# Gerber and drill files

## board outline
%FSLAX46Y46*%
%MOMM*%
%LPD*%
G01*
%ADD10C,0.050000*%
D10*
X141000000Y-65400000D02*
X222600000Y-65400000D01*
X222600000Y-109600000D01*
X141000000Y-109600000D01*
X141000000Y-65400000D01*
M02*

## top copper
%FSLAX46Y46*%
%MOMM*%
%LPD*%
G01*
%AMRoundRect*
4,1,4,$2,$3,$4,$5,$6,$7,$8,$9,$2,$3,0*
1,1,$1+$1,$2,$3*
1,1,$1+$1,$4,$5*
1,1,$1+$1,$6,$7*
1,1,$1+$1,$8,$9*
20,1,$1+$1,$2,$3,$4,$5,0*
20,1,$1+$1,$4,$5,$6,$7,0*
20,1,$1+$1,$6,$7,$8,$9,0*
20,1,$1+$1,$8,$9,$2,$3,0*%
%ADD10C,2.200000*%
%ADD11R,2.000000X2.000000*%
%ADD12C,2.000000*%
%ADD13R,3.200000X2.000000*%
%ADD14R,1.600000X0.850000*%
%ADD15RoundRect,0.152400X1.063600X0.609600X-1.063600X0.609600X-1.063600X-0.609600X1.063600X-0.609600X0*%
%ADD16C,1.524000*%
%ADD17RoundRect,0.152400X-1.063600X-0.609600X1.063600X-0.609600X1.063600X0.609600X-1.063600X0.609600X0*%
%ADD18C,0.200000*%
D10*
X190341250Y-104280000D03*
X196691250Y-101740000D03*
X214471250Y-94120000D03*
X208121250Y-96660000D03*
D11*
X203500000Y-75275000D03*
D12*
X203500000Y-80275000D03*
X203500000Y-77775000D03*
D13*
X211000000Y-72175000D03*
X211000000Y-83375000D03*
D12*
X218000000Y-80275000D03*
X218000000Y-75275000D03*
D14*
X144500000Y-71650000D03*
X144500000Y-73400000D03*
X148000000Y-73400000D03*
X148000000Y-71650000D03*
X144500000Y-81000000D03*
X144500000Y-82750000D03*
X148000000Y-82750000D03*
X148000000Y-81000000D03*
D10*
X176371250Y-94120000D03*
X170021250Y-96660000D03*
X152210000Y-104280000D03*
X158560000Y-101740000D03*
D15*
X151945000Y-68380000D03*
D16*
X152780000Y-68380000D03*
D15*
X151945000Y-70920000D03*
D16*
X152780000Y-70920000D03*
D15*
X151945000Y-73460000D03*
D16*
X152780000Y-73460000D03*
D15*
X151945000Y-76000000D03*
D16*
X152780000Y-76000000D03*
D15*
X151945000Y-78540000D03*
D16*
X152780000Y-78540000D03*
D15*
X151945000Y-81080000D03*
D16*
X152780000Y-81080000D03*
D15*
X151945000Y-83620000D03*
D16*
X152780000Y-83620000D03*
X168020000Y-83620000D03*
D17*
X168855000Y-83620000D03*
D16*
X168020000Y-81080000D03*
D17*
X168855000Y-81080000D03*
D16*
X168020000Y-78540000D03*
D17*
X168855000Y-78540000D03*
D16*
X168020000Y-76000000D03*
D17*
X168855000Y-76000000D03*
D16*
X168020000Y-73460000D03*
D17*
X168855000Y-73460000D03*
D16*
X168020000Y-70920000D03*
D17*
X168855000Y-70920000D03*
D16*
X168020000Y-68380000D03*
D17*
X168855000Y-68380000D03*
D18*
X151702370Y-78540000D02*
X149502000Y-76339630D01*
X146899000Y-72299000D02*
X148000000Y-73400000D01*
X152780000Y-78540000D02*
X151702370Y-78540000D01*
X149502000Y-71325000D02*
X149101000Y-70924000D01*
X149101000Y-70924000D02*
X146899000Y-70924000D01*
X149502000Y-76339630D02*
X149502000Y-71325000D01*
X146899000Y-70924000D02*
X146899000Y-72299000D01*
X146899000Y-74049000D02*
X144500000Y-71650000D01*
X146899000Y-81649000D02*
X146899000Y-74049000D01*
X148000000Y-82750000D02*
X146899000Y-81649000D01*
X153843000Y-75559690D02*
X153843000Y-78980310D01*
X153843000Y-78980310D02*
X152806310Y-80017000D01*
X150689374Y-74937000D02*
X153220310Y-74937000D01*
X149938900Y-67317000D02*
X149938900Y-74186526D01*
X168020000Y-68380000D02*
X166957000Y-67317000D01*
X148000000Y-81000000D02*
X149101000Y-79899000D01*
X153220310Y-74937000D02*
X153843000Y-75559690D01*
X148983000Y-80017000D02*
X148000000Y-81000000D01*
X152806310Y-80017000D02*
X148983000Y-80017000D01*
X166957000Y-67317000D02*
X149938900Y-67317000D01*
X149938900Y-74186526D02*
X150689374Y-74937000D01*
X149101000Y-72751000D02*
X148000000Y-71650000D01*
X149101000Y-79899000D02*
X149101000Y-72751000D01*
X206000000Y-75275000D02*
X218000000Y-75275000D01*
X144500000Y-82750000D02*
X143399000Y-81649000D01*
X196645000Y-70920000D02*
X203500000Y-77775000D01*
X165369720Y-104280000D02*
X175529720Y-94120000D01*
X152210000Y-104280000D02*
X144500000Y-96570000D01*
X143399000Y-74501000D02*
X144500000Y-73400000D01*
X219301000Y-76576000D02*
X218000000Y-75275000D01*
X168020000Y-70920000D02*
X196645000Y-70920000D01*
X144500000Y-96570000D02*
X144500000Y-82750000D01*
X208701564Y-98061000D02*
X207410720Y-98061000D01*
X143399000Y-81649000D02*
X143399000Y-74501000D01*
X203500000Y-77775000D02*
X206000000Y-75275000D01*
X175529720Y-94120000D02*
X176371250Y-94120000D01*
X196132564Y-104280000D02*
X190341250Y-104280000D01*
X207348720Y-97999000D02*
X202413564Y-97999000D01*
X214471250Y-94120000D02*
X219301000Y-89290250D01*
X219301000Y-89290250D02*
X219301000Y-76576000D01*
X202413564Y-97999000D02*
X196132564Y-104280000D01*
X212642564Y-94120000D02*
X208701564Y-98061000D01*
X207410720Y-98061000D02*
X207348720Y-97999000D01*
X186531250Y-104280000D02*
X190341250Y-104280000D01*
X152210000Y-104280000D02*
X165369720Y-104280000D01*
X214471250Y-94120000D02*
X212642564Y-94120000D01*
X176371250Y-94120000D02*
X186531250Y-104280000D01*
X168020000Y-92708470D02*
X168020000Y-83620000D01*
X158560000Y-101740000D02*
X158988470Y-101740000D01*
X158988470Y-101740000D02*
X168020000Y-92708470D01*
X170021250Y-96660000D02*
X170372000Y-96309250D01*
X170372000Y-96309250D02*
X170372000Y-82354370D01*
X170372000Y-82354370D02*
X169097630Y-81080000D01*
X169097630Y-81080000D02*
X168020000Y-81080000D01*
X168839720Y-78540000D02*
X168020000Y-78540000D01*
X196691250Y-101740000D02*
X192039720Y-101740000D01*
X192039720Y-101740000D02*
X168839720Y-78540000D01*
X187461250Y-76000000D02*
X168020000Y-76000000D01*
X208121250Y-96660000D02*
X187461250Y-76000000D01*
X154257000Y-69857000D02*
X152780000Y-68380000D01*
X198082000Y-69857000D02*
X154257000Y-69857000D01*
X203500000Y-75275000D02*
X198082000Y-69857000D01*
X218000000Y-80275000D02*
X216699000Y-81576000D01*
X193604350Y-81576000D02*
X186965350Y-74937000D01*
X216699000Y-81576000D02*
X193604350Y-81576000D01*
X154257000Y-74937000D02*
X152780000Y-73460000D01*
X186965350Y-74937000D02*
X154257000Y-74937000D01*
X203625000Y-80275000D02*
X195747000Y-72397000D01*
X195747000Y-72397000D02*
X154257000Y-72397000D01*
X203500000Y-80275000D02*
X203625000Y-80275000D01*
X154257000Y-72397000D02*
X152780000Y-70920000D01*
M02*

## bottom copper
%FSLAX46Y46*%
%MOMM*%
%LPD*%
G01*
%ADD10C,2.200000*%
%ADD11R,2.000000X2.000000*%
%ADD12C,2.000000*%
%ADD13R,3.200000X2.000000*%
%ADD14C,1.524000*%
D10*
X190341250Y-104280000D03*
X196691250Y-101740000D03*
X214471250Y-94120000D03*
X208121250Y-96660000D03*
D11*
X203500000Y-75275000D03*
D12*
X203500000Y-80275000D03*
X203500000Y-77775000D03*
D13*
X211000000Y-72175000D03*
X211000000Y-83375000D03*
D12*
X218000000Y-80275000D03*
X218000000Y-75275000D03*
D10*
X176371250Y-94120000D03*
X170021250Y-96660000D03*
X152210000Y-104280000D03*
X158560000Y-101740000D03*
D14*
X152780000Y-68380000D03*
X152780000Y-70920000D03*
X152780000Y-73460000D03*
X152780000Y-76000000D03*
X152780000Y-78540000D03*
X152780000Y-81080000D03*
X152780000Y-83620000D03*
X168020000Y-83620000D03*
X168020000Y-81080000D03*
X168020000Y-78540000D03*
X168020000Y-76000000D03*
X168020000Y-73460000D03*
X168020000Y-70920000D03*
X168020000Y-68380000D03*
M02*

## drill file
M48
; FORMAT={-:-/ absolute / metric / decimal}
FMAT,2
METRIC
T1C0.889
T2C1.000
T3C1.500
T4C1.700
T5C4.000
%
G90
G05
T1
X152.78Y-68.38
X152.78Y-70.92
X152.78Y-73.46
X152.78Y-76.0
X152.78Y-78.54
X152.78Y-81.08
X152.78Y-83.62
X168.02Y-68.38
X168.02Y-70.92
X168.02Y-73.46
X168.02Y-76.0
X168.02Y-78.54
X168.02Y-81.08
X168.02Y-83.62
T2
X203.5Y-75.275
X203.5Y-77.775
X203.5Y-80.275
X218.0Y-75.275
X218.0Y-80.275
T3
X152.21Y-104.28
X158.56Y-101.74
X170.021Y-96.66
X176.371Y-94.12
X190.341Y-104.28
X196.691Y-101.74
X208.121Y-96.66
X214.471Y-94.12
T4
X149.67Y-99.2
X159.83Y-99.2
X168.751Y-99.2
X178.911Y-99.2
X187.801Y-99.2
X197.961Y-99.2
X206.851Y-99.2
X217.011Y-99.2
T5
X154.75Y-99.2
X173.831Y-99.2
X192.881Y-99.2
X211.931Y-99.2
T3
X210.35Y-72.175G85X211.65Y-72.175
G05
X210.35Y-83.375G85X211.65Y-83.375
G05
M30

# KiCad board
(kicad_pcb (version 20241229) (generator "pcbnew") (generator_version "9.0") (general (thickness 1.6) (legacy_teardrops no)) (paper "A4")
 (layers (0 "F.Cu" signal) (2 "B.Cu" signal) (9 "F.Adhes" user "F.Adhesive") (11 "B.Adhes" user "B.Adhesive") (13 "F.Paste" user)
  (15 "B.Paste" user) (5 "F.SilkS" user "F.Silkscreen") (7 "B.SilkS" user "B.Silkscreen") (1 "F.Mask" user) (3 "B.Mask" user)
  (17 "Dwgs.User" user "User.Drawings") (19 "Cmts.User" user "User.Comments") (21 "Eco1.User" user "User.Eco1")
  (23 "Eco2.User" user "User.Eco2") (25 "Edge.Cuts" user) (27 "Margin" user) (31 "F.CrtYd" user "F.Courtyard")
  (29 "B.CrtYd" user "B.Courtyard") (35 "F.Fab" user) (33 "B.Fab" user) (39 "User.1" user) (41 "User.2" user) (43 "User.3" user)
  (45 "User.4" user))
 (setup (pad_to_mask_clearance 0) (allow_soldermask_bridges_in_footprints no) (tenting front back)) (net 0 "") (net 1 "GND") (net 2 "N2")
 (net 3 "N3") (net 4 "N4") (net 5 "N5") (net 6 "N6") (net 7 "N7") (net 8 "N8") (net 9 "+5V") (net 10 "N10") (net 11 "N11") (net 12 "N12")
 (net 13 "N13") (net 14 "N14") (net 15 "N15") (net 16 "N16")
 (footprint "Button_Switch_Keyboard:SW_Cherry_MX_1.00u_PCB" (layer "F.Cu") (at 190.34125 104.28 180)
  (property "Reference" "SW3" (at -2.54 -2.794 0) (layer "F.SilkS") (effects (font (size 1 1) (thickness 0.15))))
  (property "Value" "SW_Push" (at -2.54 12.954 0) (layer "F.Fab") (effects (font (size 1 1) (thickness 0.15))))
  (pad "" np_thru_hole circle (at -7.62 5.08 180) (size 1.7 1.7) (drill 1.7) (layers "*.Cu" "*.Mask"))
  (pad "" np_thru_hole circle (at -2.54 5.08 180) (size 4 4) (drill 4) (layers "*.Cu" "*.Mask"))
  (pad "" np_thru_hole circle (at 2.54 5.08 180) (size 1.7 1.7) (drill 1.7) (layers "*.Cu" "*.Mask"))
  (pad "1" thru_hole circle (at 0 0 180) (size 2.2 2.2) (drill 1.5) (layers "*.Cu" "*.Mask") (remove_unused_layers no) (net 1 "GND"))
  (pad "2" thru_hole circle (at -6.35 2.54 180) (size 2.2 2.2) (drill 1.5) (layers "*.Cu" "*.Mask") (remove_unused_layers no) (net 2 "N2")))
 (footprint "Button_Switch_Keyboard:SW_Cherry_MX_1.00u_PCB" (layer "F.Cu") (at 214.47125 94.12)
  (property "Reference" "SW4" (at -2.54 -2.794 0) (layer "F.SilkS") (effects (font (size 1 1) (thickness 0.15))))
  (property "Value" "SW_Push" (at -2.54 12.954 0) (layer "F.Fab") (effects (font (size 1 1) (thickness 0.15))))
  (pad "" np_thru_hole circle (at -7.62 5.08) (size 1.7 1.7) (drill 1.7) (layers "*.Cu" "*.Mask"))
  (pad "" np_thru_hole circle (at -2.54 5.08) (size 4 4) (drill 4) (layers "*.Cu" "*.Mask"))
  (pad "" np_thru_hole circle (at 2.54 5.08) (size 1.7 1.7) (drill 1.7) (layers "*.Cu" "*.Mask"))
  (pad "1" thru_hole circle (at 0 0) (size 2.2 2.2) (drill 1.5) (layers "*.Cu" "*.Mask") (remove_unused_layers no) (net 1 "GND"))
  (pad "2" thru_hole circle (at -6.35 2.54) (size 2.2 2.2) (drill 1.5) (layers "*.Cu" "*.Mask") (remove_unused_layers no) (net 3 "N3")))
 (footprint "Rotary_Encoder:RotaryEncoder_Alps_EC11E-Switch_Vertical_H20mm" (layer "F.Cu") (at 203.5 75.275)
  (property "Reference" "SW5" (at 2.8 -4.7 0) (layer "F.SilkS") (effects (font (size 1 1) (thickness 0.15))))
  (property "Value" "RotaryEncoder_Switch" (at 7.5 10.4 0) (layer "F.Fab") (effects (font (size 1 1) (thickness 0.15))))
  (pad "A" thru_hole rect (at 0 0) (size 2 2) (drill 1) (layers "*.Cu" "*.Mask") (remove_unused_layers no) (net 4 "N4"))
  (pad "B" thru_hole circle (at 0 5) (size 2 2) (drill 1) (layers "*.Cu" "*.Mask") (remove_unused_layers no) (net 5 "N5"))
  (pad "C" thru_hole circle (at 0 2.5) (size 2 2) (drill 1) (layers "*.Cu" "*.Mask") (remove_unused_layers no) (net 1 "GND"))
  (pad "MP" thru_hole rect (at 7.5 -3.1) (size 3.2 2) (drill oval 2.8 1.5) (layers "*.Cu" "*.Mask") (remove_unused_layers no))
  (pad "MP" thru_hole rect (at 7.5 8.1) (size 3.2 2) (drill oval 2.8 1.5) (layers "*.Cu" "*.Mask") (remove_unused_layers no))
  (pad "S1" thru_hole circle (at 14.5 5) (size 2 2) (drill 1) (layers "*.Cu" "*.Mask") (remove_unused_layers no) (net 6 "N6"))
  (pad "S2" thru_hole circle (at 14.5 0) (size 2 2) (drill 1) (layers "*.Cu" "*.Mask") (remove_unused_layers no) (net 1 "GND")))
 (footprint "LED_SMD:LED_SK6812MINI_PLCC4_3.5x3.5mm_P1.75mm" (layer "F.Cu") (at 146.25 72.525)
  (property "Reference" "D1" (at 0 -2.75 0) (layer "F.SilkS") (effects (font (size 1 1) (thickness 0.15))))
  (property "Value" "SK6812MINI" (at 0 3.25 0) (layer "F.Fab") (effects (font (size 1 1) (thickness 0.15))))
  (pad "1" smd rect (at -1.75 -0.875) (size 1.6 0.85) (layers "F.Cu" "F.Mask" "F.Paste") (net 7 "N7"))
  (pad "2" smd rect (at -1.75 0.875) (size 1.6 0.85) (layers "F.Cu" "F.Mask" "F.Paste") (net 1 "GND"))
  (pad "3" smd rect (at 1.75 0.875) (size 1.6 0.85) (layers "F.Cu" "F.Mask" "F.Paste") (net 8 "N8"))
  (pad "4" smd rect (at 1.75 -0.875) (size 1.6 0.85) (layers "F.Cu" "F.Mask" "F.Paste") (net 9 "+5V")))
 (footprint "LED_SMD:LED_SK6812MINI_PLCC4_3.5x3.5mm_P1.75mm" (layer "F.Cu") (at 146.25 81.875)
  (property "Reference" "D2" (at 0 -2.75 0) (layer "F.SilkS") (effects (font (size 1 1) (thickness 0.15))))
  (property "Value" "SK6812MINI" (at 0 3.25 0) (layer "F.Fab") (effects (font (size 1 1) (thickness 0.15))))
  (pad "1" smd rect (at -1.75 -0.875) (size 1.6 0.85) (layers "F.Cu" "F.Mask" "F.Paste") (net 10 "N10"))
  (pad "2" smd rect (at -1.75 0.875) (size 1.6 0.85) (layers "F.Cu" "F.Mask" "F.Paste") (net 1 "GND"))
  (pad "3" smd rect (at 1.75 0.875) (size 1.6 0.85) (layers "F.Cu" "F.Mask" "F.Paste") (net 7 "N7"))
  (pad "4" smd rect (at 1.75 -0.875) (size 1.6 0.85) (layers "F.Cu" "F.Mask" "F.Paste") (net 9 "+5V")))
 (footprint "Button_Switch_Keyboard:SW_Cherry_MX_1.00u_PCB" (layer "F.Cu") (at 176.37125 94.12)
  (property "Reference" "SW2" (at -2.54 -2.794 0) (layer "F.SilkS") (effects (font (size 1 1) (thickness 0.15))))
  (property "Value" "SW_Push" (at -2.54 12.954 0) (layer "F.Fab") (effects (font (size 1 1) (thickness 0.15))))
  (pad "" np_thru_hole circle (at -7.62 5.08) (size 1.7 1.7) (drill 1.7) (layers "*.Cu" "*.Mask"))
  (pad "" np_thru_hole circle (at -2.54 5.08) (size 4 4) (drill 4) (layers "*.Cu" "*.Mask"))
  (pad "" np_thru_hole circle (at 2.54 5.08) (size 1.7 1.7) (drill 1.7) (layers "*.Cu" "*.Mask"))
  (pad "1" thru_hole circle (at 0 0) (size 2.2 2.2) (drill 1.5) (layers "*.Cu" "*.Mask") (remove_unused_layers no) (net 1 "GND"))
  (pad "2" thru_hole circle (at -6.35 2.54) (size 2.2 2.2) (drill 1.5) (layers "*.Cu" "*.Mask") (remove_unused_layers no) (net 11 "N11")))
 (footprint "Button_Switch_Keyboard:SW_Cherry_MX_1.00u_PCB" (layer "F.Cu") (at 152.21 104.28 180)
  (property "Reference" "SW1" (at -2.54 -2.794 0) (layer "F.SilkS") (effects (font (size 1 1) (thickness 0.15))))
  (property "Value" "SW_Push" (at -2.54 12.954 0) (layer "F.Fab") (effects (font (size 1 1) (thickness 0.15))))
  (pad "" np_thru_hole circle (at -7.62 5.08 180) (size 1.7 1.7) (drill 1.7) (layers "*.Cu" "*.Mask"))
  (pad "" np_thru_hole circle (at -2.54 5.08 180) (size 4 4) (drill 4) (layers "*.Cu" "*.Mask"))
  (pad "" np_thru_hole circle (at 2.54 5.08 180) (size 1.7 1.7) (drill 1.7) (layers "*.Cu" "*.Mask"))
  (pad "1" thru_hole circle (at 0 0 180) (size 2.2 2.2) (drill 1.5) (layers "*.Cu" "*.Mask") (remove_unused_layers no) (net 1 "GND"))
  (pad "2" thru_hole circle (at -6.35 2.54 180) (size 2.2 2.2) (drill 1.5) (layers "*.Cu" "*.Mask") (remove_unused_layers no) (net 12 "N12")))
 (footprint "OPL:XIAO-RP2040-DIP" (layer "F.Cu") (at 160.4 76)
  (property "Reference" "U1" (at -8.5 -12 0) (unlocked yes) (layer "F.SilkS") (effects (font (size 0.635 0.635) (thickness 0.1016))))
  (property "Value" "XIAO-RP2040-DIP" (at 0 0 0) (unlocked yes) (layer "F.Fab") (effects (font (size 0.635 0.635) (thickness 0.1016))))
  (pad "1" smd roundrect (at -8.455 -7.62 180) (size 2.432 1.524) (layers "F.Cu" "F.Mask") (roundrect_rratio 0.1) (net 4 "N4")
   (thermal_bridge_angle 45))
  (pad "1" thru_hole circle (at -7.62 -7.62 180) (size 1.524 1.524) (drill 0.889) (layers "*.Cu" "*.Mask") (remove_unused_layers no)
   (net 4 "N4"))
  (pad "2" smd roundrect (at -8.455 -5.08 180) (size 2.432 1.524) (layers "F.Cu" "F.Mask") (roundrect_rratio 0.1) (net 5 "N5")
   (thermal_bridge_angle 45))
  (pad "2" thru_hole circle (at -7.62 -5.08 180) (size 1.524 1.524) (drill 0.889) (layers "*.Cu" "*.Mask") (remove_unused_layers no)
   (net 5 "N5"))
  (pad "3" smd roundrect (at -8.455 -2.54 180) (size 2.432 1.524) (layers "F.Cu" "F.Mask") (roundrect_rratio 0.1) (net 6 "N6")
   (thermal_bridge_angle 45))
  (pad "3" thru_hole circle (at -7.62 -2.54 180) (size 1.524 1.524) (drill 0.889) (layers "*.Cu" "*.Mask") (remove_unused_layers no)
   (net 6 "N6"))
  (pad "4" smd roundrect (at -8.455 0 180) (size 2.432 1.524) (layers "F.Cu" "F.Mask") (roundrect_rratio 0.1) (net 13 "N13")
   (thermal_bridge_angle 45))
  (pad "4" thru_hole circle (at -7.62 0 180) (size 1.524 1.524) (drill 0.889) (layers "*.Cu" "*.Mask") (remove_unused_layers no)
   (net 13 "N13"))
  (pad "5" smd roundrect (at -8.455 2.54 180) (size 2.432 1.524) (layers "F.Cu" "F.Mask") (roundrect_rratio 0.1) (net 8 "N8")
   (thermal_bridge_angle 45))
  (pad "5" thru_hole circle (at -7.62 2.54 180) (size 1.524 1.524) (drill 0.889) (layers "*.Cu" "*.Mask") (remove_unused_layers no)
   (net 8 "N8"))
  (pad "6" smd roundrect (at -8.455 5.08 180) (size 2.432 1.524) (layers "F.Cu" "F.Mask") (roundrect_rratio 0.1) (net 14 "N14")
   (thermal_bridge_angle 45))
  (pad "6" thru_hole circle (at -7.62 5.08 180) (size 1.524 1.524) (drill 0.889) (layers "*.Cu" "*.Mask") (remove_unused_layers no)
   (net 14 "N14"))
  (pad "7" smd roundrect (at -8.455 7.62 180) (size 2.432 1.524) (layers "F.Cu" "F.Mask") (roundrect_rratio 0.1) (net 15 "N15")
   (thermal_bridge_angle 45))
  (pad "7" thru_hole circle (at -7.62 7.62 180) (size 1.524 1.524) (drill 0.889) (layers "*.Cu" "*.Mask") (remove_unused_layers no)
   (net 15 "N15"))
  (pad "8" thru_hole circle (at 7.62 7.62) (size 1.524 1.524) (drill 0.889) (layers "*.Cu" "*.Mask") (remove_unused_layers no)
   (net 12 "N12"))
  (pad "8" smd roundrect (at 8.455 7.62) (size 2.432 1.524) (layers "F.Cu" "F.Mask") (roundrect_rratio 0.1) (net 12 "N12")
   (thermal_bridge_angle 45))
  (pad "9" thru_hole circle (at 7.62 5.08) (size 1.524 1.524) (drill 0.889) (layers "*.Cu" "*.Mask") (remove_unused_layers no)
   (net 11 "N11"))
  (pad "9" smd roundrect (at 8.455 5.08) (size 2.432 1.524) (layers "F.Cu" "F.Mask") (roundrect_rratio 0.1) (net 11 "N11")
   (thermal_bridge_angle 45))
  (pad "10" thru_hole circle (at 7.62 2.54) (size 1.524 1.524) (drill 0.889) (layers "*.Cu" "*.Mask") (remove_unused_layers no) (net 2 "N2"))
  (pad "10" smd roundrect (at 8.455 2.54) (size 2.432 1.524) (layers "F.Cu" "F.Mask") (roundrect_rratio 0.1) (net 2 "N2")
   (thermal_bridge_angle 45))
  (pad "11" thru_hole circle (at 7.62 0) (size 1.524 1.524) (drill 0.889) (layers "*.Cu" "*.Mask") (remove_unused_layers no) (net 3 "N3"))
  (pad "11" smd roundrect (at 8.455 0) (size 2.432 1.524) (layers "F.Cu" "F.Mask") (roundrect_rratio 0.1) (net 3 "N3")
   (thermal_bridge_angle 45))
  (pad "12" thru_hole circle (at 7.62 -2.54) (size 1.524 1.524) (drill 0.889) (layers "*.Cu" "*.Mask") (remove_unused_layers no)
   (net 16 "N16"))
  (pad "12" smd roundrect (at 8.455 -2.54) (size 2.432 1.524) (layers "F.Cu" "F.Mask") (roundrect_rratio 0.1) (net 16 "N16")
   (thermal_bridge_angle 45))
  (pad "13" thru_hole circle (at 7.62 -5.08) (size 1.524 1.524) (drill 0.889) (layers "*.Cu" "*.Mask") (remove_unused_layers no)
   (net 1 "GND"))
  (pad "13" smd roundrect (at 8.455 -5.08) (size 2.432 1.524) (layers "F.Cu" "F.Mask") (roundrect_rratio 0.1) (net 1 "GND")
   (thermal_bridge_angle 45))
  (pad "14" thru_hole circle (at 7.62 -7.62) (size 1.524 1.524) (drill 0.889) (layers "*.Cu" "*.Mask") (remove_unused_layers no)
   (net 9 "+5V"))
  (pad "14" smd roundrect (at 8.455 -7.62) (size 2.432 1.524) (layers "F.Cu" "F.Mask") (roundrect_rratio 0.1) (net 9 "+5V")
   (thermal_bridge_angle 45)))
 (gr_rect (start 141 65.4) (end 222.6 109.6) (stroke (width 0.05) (type default)) (fill no) (layer "Edge.Cuts"))
 (segment (start 151.70237 78.54) (end 149.502 76.33963) (width 0.2) (layer "F.Cu") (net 8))
 (segment (start 146.899 72.299) (end 148 73.4) (width 0.2) (layer "F.Cu") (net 8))
 (segment (start 152.78 78.54) (end 151.70237 78.54) (width 0.2) (layer "F.Cu") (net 8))
 (segment (start 149.502 71.325) (end 149.101 70.924) (width 0.2) (layer "F.Cu") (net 8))
 (segment (start 149.101 70.924) (end 146.899 70.924) (width 0.2) (layer "F.Cu") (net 8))
 (segment (start 149.502 76.33963) (end 149.502 71.325) (width 0.2) (layer "F.Cu") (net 8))
 (segment (start 146.899 70.924) (end 146.899 72.299) (width 0.2) (layer "F.Cu") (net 8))
 (segment (start 146.899 74.049) (end 144.5 71.65) (width 0.2) (layer "F.Cu") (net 7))
 (segment (start 146.899 81.649) (end 146.899 74.049) (width 0.2) (layer "F.Cu") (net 7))
 (segment (start 148 82.75) (end 146.899 81.649) (width 0.2) (layer "F.Cu") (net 7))
 (segment (start 153.843 75.55969) (end 153.843 78.98031) (width 0.2) (layer "F.Cu") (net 9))
 (segment (start 153.843 78.98031) (end 152.80631 80.017) (width 0.2) (layer "F.Cu") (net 9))
 (segment (start 150.689374 74.937) (end 153.22031 74.937) (width 0.2) (layer "F.Cu") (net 9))
 (segment (start 149.9389 67.317) (end 149.9389 74.186526) (width 0.2) (layer "F.Cu") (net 9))
 (segment (start 168.02 68.38) (end 166.957 67.317) (width 0.2) (layer "F.Cu") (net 9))
 (segment (start 148 81) (end 149.101 79.899) (width 0.2) (layer "F.Cu") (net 9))
 (segment (start 153.22031 74.937) (end 153.843 75.55969) (width 0.2) (layer "F.Cu") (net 9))
 (segment (start 148.983 80.017) (end 148 81) (width 0.2) (layer "F.Cu") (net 9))
 (segment (start 152.80631 80.017) (end 148.983 80.017) (width 0.2) (layer "F.Cu") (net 9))
 (segment (start 166.957 67.317) (end 149.9389 67.317) (width 0.2) (layer "F.Cu") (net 9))
 (segment (start 149.9389 74.186526) (end 150.689374 74.937) (width 0.2) (layer "F.Cu") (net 9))
 (segment (start 149.101 72.751) (end 148 71.65) (width 0.2) (layer "F.Cu") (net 9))
 (segment (start 149.101 79.899) (end 149.101 72.751) (width 0.2) (layer "F.Cu") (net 9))
 (segment (start 206 75.275) (end 218 75.275) (width 0.2) (layer "F.Cu") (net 1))
 (segment (start 144.5 82.75) (end 143.399 81.649) (width 0.2) (layer "F.Cu") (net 1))
 (segment (start 196.645 70.92) (end 203.5 77.775) (width 0.2) (layer "F.Cu") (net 1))
 (segment (start 165.36972 104.28) (end 175.52972 94.12) (width 0.2) (layer "F.Cu") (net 1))
 (segment (start 152.21 104.28) (end 144.5 96.57) (width 0.2) (layer "F.Cu") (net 1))
 (segment (start 143.399 74.501) (end 144.5 73.4) (width 0.2) (layer "F.Cu") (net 1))
 (segment (start 219.301 76.576) (end 218 75.275) (width 0.2) (layer "F.Cu") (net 1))
 (segment (start 168.02 70.92) (end 196.645 70.92) (width 0.2) (layer "F.Cu") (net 1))
 (segment (start 144.5 96.57) (end 144.5 82.75) (width 0.2) (layer "F.Cu") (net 1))
 (segment (start 208.701564 98.061) (end 207.41072 98.061) (width 0.2) (layer "F.Cu") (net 1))
 (segment (start 143.399 81.649) (end 143.399 74.501) (width 0.2) (layer "F.Cu") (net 1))
 (segment (start 203.5 77.775) (end 206 75.275) (width 0.2) (layer "F.Cu") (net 1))
 (segment (start 175.52972 94.12) (end 176.37125 94.12) (width 0.2) (layer "F.Cu") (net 1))
 (segment (start 196.132564 104.28) (end 190.34125 104.28) (width 0.2) (layer "F.Cu") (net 1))
 (segment (start 207.34872 97.999) (end 202.413564 97.999) (width 0.2) (layer "F.Cu") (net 1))
 (segment (start 214.47125 94.12) (end 219.301 89.29025) (width 0.2) (layer "F.Cu") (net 1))
 (segment (start 219.301 89.29025) (end 219.301 76.576) (width 0.2) (layer "F.Cu") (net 1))
 (segment (start 202.413564 97.999) (end 196.132564 104.28) (width 0.2) (layer "F.Cu") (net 1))
 (segment (start 212.642564 94.12) (end 208.701564 98.061) (width 0.2) (layer "F.Cu") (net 1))
 (segment (start 207.41072 98.061) (end 207.34872 97.999) (width 0.2) (layer "F.Cu") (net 1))
 (segment (start 186.53125 104.28) (end 190.34125 104.28) (width 0.2) (layer "F.Cu") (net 1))
 (segment (start 152.21 104.28) (end 165.36972 104.28) (width 0.2) (layer "F.Cu") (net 1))
 (segment (start 214.47125 94.12) (end 212.642564 94.12) (width 0.2) (layer "F.Cu") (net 1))
 (segment (start 176.37125 94.12) (end 186.53125 104.28) (width 0.2) (layer "F.Cu") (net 1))
 (segment (start 168.02 92.70847) (end 168.02 83.62) (width 0.2) (layer "F.Cu") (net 12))
 (segment (start 158.56 101.74) (end 158.98847 101.74) (width 0.2) (layer "F.Cu") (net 12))
 (segment (start 158.98847 101.74) (end 168.02 92.70847) (width 0.2) (layer "F.Cu") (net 12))
 (segment (start 170.02125 96.66) (end 170.372 96.30925) (width 0.2) (layer "F.Cu") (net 11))
 (segment (start 170.372 96.30925) (end 170.372 82.35437) (width 0.2) (layer "F.Cu") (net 11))
 (segment (start 170.372 82.35437) (end 169.09763 81.08) (width 0.2) (layer "F.Cu") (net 11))
 (segment (start 169.09763 81.08) (end 168.02 81.08) (width 0.2) (layer "F.Cu") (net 11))
 (segment (start 168.83972 78.54) (end 168.02 78.54) (width 0.2) (layer "F.Cu") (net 2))
 (segment (start 196.69125 101.74) (end 192.03972 101.74) (width 0.2) (layer "F.Cu") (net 2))
 (segment (start 192.03972 101.74) (end 168.83972 78.54) (width 0.2) (layer "F.Cu") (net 2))
 (segment (start 187.46125 76) (end 168.02 76) (width 0.2) (layer "F.Cu") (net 3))
 (segment (start 208.12125 96.66) (end 187.46125 76) (width 0.2) (layer "F.Cu") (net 3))
 (segment (start 154.257 69.857) (end 152.78 68.38) (width 0.2) (layer "F.Cu") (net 4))
 (segment (start 198.082 69.857) (end 154.257 69.857) (width 0.2) (layer "F.Cu") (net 4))
 (segment (start 203.5 75.275) (end 198.082 69.857) (width 0.2) (layer "F.Cu") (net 4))
 (segment (start 218 80.275) (end 216.699 81.576) (width 0.2) (layer "F.Cu") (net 6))
 (segment (start 193.60435 81.576) (end 186.96535 74.937) (width 0.2) (layer "F.Cu") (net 6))
 (segment (start 216.699 81.576) (end 193.60435 81.576) (width 0.2) (layer "F.Cu") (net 6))
 (segment (start 154.257 74.937) (end 152.78 73.46) (width 0.2) (layer "F.Cu") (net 6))
 (segment (start 186.96535 74.937) (end 154.257 74.937) (width 0.2) (layer "F.Cu") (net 6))
 (segment (start 203.625 80.275) (end 195.747 72.397) (width 0.2) (layer "F.Cu") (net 5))
 (segment (start 195.747 72.397) (end 154.257 72.397) (width 0.2) (layer "F.Cu") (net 5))
 (segment (start 203.5 80.275) (end 203.625 80.275) (width 0.2) (layer "F.Cu") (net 5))
 (segment (start 154.257 72.397) (end 152.78 70.92) (width 0.2) (layer "F.Cu") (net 5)))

